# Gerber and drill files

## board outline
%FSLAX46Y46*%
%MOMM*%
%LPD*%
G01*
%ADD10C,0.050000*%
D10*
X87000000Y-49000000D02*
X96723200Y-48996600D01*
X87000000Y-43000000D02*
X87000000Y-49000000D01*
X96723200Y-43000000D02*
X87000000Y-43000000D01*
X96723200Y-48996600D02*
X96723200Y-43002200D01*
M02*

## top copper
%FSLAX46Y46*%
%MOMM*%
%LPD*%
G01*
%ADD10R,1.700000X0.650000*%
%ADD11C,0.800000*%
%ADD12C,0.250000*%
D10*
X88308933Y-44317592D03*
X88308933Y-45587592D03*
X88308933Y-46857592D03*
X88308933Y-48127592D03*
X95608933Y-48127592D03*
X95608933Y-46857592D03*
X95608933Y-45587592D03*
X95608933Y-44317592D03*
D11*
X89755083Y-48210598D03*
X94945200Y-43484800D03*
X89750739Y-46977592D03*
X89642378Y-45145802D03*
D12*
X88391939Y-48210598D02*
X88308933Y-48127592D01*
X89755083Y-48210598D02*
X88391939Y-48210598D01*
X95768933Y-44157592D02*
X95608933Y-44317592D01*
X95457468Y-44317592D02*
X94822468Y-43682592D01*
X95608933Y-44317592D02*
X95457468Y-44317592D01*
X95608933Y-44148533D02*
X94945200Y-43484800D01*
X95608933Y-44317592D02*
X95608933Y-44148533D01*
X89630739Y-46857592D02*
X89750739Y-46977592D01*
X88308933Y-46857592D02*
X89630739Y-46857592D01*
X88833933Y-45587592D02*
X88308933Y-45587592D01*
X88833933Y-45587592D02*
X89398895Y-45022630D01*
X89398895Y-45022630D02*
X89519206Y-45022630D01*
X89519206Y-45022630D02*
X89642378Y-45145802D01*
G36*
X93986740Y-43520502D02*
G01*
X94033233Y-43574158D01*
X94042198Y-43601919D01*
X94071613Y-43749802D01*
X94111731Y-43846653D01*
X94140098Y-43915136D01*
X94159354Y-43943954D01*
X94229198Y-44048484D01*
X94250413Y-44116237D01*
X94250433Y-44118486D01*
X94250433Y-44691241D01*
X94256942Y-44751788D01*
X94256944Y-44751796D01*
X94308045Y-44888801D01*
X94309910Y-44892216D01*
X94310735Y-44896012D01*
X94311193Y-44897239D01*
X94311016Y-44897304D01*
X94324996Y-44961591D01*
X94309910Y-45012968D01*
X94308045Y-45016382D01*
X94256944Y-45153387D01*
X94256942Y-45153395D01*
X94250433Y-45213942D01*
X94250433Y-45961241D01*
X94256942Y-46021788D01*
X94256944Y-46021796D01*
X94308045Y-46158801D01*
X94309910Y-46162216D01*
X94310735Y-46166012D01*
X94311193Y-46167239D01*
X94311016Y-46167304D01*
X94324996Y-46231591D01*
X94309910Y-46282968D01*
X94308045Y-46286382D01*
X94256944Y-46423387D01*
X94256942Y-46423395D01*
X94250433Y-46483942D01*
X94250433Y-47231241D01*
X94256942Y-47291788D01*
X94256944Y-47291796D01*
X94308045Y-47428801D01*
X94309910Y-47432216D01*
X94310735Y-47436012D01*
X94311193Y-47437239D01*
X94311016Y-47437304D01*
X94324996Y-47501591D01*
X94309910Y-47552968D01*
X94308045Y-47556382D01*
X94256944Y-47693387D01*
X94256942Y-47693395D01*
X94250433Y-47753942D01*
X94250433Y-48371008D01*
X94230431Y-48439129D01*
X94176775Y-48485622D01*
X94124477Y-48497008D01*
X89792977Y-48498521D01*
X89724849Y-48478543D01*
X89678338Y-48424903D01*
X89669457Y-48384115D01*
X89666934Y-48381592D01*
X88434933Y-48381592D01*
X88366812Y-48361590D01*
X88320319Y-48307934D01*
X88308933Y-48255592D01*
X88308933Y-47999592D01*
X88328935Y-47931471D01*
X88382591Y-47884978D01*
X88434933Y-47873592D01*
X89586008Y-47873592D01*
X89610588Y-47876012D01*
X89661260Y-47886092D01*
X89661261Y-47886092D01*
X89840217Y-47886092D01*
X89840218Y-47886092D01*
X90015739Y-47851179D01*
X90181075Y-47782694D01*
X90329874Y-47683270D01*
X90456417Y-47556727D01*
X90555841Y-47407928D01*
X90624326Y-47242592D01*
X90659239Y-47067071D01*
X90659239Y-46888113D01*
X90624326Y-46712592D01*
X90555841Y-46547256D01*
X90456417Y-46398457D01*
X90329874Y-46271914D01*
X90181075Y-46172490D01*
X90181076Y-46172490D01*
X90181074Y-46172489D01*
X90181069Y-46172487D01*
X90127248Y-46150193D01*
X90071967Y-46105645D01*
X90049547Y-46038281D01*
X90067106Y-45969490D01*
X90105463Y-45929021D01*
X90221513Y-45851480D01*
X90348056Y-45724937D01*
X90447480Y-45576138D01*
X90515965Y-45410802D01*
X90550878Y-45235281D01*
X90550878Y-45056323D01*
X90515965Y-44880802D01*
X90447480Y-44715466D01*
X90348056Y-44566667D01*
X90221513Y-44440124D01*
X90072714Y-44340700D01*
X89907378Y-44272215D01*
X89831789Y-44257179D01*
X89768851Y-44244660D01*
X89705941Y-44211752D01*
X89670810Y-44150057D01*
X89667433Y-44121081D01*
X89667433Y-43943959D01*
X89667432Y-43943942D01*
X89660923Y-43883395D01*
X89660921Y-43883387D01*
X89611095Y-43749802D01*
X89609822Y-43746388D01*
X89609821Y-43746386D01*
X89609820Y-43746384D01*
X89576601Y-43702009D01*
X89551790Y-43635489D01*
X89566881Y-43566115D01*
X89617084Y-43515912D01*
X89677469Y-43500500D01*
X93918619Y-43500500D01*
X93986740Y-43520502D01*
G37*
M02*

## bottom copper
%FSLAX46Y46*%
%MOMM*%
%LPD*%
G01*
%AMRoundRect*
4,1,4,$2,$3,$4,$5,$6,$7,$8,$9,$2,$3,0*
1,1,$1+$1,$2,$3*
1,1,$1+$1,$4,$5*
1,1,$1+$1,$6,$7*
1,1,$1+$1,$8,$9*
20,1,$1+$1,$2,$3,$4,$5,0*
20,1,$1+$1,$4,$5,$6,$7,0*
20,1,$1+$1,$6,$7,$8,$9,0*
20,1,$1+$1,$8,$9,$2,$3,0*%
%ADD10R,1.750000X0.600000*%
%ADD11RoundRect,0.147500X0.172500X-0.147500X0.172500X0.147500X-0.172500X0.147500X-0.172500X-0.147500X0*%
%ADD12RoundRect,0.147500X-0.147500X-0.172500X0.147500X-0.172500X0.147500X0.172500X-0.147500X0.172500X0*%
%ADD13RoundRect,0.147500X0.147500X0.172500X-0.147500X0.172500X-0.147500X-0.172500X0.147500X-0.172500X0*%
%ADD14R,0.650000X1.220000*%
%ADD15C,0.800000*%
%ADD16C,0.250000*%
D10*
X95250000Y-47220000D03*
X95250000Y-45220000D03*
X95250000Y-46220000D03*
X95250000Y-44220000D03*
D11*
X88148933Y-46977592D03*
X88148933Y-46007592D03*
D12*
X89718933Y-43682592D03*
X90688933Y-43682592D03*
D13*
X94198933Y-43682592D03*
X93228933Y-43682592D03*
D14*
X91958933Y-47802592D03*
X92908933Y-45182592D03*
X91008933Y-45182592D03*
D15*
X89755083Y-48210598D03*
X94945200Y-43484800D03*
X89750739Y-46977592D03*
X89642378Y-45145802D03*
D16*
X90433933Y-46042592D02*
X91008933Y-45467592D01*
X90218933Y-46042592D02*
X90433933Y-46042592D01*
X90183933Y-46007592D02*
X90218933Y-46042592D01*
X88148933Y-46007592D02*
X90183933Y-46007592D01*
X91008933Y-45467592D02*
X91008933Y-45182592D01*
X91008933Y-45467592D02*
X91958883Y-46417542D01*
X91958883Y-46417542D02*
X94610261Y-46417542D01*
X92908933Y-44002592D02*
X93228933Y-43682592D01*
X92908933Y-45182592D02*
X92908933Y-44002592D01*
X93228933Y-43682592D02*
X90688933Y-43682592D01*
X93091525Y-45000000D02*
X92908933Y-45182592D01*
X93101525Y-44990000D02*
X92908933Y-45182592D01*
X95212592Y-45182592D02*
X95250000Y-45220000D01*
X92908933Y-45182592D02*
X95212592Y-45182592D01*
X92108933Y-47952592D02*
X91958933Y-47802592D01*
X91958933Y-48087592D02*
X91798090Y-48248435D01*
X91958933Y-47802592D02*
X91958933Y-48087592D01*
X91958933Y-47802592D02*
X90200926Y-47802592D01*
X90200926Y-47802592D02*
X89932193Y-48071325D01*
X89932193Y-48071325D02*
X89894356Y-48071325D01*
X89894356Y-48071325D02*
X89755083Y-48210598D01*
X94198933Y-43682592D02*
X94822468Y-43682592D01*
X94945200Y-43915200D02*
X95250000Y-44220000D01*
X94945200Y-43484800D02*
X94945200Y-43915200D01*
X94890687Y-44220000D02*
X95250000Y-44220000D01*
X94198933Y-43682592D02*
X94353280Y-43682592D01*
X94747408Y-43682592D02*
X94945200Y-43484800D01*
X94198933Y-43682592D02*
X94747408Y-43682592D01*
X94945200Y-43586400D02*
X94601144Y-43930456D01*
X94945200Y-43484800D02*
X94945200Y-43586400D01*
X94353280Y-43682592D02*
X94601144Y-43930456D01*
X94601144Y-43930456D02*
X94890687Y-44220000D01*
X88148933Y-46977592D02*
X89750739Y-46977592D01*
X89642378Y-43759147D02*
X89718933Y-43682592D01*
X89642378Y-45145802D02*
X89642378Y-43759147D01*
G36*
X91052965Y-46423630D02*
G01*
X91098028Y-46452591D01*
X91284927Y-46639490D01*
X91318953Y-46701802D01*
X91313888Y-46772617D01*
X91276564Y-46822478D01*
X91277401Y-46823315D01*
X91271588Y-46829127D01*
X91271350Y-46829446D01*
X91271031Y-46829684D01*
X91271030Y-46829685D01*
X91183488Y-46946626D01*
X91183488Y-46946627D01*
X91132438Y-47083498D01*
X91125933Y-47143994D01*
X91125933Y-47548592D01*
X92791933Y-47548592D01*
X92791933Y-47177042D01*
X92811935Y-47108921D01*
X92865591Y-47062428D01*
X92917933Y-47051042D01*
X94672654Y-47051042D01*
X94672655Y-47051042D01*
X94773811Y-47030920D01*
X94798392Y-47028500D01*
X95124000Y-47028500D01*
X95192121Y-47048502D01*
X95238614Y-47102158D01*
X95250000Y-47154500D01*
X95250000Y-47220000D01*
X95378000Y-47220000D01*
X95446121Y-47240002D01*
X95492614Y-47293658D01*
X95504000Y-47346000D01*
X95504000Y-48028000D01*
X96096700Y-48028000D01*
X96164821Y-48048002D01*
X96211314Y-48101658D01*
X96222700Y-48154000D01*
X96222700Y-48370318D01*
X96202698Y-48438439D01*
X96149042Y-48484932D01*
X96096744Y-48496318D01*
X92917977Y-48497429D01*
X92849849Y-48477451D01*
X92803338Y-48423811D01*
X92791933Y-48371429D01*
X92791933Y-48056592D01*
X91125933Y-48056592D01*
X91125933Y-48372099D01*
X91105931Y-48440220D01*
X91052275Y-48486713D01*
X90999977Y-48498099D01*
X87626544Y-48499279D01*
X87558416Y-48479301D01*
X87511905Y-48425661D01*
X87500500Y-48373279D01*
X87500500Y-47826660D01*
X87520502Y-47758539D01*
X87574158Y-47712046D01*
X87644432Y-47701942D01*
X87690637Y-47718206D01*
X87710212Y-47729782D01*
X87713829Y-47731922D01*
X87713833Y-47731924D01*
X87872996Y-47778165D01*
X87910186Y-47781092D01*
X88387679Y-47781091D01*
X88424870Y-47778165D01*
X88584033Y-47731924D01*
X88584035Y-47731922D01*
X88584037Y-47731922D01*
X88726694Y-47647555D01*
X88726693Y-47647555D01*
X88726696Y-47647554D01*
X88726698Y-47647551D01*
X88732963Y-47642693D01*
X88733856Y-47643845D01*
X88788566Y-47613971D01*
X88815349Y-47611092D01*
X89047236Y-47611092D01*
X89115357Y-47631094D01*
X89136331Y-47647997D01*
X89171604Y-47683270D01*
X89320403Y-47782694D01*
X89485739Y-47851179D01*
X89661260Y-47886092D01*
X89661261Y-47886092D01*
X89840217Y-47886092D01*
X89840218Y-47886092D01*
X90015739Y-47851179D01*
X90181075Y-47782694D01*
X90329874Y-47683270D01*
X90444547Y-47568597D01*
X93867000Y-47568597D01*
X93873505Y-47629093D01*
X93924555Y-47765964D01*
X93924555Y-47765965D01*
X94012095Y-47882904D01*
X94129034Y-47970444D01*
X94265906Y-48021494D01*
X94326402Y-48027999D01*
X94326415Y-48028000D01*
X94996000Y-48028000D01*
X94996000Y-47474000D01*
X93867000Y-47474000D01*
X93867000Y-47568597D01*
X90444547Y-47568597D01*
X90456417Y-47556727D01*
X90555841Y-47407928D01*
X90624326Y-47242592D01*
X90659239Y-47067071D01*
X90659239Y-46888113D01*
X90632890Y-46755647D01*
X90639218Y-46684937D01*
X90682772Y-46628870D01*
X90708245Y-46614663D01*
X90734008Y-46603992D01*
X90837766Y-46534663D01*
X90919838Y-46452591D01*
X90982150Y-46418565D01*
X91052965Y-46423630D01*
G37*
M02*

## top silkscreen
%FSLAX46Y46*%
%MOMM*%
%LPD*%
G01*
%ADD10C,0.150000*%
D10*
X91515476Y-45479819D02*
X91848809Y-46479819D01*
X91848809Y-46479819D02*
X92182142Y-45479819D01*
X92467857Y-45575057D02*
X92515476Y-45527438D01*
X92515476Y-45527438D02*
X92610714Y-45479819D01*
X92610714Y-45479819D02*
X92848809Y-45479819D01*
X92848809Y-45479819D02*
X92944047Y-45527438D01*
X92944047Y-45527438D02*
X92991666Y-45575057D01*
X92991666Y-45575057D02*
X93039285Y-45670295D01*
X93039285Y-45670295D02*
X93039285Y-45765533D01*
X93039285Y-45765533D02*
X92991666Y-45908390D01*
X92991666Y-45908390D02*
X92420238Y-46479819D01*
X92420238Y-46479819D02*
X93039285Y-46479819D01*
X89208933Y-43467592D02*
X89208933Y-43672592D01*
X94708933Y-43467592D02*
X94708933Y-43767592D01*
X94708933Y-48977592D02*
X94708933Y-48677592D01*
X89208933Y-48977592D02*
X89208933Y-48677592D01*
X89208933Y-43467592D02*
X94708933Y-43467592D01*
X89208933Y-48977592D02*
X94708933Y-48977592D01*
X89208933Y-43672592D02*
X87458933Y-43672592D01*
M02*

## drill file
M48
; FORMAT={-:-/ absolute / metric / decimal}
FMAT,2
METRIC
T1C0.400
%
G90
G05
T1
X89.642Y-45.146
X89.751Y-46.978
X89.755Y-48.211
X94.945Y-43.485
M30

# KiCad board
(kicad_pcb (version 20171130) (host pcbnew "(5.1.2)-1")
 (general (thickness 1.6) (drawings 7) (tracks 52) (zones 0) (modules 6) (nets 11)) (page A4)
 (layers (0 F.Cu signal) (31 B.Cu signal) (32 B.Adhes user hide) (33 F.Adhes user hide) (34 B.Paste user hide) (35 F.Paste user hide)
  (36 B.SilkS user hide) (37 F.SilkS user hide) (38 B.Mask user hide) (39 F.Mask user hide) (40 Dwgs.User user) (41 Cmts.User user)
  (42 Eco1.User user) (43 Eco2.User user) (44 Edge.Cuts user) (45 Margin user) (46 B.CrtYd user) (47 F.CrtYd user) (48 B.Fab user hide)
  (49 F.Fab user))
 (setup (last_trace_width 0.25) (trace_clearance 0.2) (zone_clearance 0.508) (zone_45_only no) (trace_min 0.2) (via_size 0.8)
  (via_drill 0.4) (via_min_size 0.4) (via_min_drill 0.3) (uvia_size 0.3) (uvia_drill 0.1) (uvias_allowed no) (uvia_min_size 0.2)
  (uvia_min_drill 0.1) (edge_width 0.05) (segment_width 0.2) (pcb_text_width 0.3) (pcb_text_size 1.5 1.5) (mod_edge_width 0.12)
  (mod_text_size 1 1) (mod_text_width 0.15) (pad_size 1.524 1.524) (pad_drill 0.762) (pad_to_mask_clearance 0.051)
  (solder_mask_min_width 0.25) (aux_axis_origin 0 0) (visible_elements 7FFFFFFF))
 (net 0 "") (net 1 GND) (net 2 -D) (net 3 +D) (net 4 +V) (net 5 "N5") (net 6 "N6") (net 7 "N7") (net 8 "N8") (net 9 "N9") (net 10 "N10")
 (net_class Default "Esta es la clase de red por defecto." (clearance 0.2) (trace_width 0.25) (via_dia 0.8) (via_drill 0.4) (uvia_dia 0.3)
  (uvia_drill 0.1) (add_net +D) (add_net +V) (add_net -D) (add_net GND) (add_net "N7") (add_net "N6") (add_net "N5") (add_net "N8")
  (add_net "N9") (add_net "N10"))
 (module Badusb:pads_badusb (layer B.Cu) (at 93.98 45.72 180)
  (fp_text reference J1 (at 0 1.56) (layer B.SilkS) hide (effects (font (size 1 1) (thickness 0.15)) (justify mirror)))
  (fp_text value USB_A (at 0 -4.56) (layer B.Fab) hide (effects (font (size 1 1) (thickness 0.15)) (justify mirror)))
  (pad 4 smd rect (at -1.27 -1.5 180) (size 1.75 0.6) (layers B.Cu B.Paste B.Mask) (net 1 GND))
  (pad 2 smd rect (at -1.27 0.5 180) (size 1.75 0.6) (layers B.Cu B.Paste B.Mask) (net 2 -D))
  (pad 3 smd rect (at -1.27 -0.5 180) (size 1.75 0.6) (layers B.Cu B.Paste B.Mask) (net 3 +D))
  (pad 1 smd rect (at -1.27 1.5 180) (size 1.75 0.6) (layers B.Cu B.Paste B.Mask) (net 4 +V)))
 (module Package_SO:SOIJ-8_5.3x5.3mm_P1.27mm (layer F.Cu) (at 91.958933 46.222592)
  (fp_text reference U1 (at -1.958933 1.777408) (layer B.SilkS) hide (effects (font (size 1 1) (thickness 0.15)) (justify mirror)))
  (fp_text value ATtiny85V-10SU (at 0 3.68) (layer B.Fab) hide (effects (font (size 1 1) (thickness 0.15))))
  (fp_line (start -2.75 -2.755) (end -2.75 -2.55) (layer F.SilkS) (width 0.15))
  (fp_line (start 2.75 -2.755) (end 2.75 -2.455) (layer F.SilkS) (width 0.15))
  (fp_line (start 2.75 2.755) (end 2.75 2.455) (layer F.SilkS) (width 0.15))
  (fp_line (start -2.75 2.755) (end -2.75 2.455) (layer F.SilkS) (width 0.15))
  (fp_line (start -2.75 -2.755) (end 2.75 -2.755) (layer F.SilkS) (width 0.15))
  (fp_line (start -2.75 2.755) (end 2.75 2.755) (layer F.SilkS) (width 0.15))
  (fp_line (start -2.75 -2.55) (end -4.5 -2.55) (layer F.SilkS) (width 0.15))
  (pad 1 smd rect (at -3.65 -1.905) (size 1.7 0.65) (layers F.Cu F.Paste F.Mask) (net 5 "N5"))
  (pad 2 smd rect (at -3.65 -0.635) (size 1.7 0.65) (layers F.Cu F.Paste F.Mask) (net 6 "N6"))
  (pad 3 smd rect (at -3.65 0.635) (size 1.7 0.65) (layers F.Cu F.Paste F.Mask) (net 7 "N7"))
  (pad 4 smd rect (at -3.65 1.905) (size 1.7 0.65) (layers F.Cu F.Paste F.Mask) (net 1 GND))
  (pad 5 smd rect (at 3.65 1.905) (size 1.7 0.65) (layers F.Cu F.Paste F.Mask) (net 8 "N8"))
  (pad 6 smd rect (at 3.65 0.635) (size 1.7 0.65) (layers F.Cu F.Paste F.Mask) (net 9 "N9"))
  (pad 7 smd rect (at 3.65 -0.635) (size 1.7 0.65) (layers F.Cu F.Paste F.Mask) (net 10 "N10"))
  (pad 8 smd rect (at 3.65 -1.905) (size 1.7 0.65) (layers F.Cu F.Paste F.Mask) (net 4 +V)))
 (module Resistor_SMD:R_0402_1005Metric (layer B.Cu) (at 88.148933 46.492592 90)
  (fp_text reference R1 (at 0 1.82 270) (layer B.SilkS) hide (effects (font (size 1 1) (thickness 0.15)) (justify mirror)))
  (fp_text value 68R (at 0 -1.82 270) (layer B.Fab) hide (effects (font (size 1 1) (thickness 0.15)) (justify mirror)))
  (pad 1 smd roundrect (at -0.485 0 90) (size 0.59 0.64) (layers B.Cu B.Paste B.Mask) (roundrect_rratio 0.25) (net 7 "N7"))
  (pad 2 smd roundrect (at 0.485 0 90) (size 0.59 0.64) (layers B.Cu B.Paste B.Mask) (roundrect_rratio 0.25) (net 3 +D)))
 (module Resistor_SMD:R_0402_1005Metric (layer B.Cu) (at 90.203933 43.682592)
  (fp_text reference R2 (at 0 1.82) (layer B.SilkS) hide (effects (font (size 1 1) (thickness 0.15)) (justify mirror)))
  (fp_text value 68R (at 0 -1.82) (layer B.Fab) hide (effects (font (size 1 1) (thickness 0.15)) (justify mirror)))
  (pad 1 smd roundrect (at -0.485 0) (size 0.59 0.64) (layers B.Cu B.Paste B.Mask) (roundrect_rratio 0.25) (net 6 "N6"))
  (pad 2 smd roundrect (at 0.485 0) (size 0.59 0.64) (layers B.Cu B.Paste B.Mask) (roundrect_rratio 0.25) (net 2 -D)))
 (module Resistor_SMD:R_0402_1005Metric (layer B.Cu) (at 93.713933 43.682592 180)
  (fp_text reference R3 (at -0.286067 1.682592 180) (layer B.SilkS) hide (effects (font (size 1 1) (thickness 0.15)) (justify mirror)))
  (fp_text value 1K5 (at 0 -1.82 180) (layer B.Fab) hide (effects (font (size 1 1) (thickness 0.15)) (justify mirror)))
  (pad 1 smd roundrect (at -0.485 0 180) (size 0.59 0.64) (layers B.Cu B.Paste B.Mask) (roundrect_rratio 0.25) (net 4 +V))
  (pad 2 smd roundrect (at 0.485 0 180) (size 0.59 0.64) (layers B.Cu B.Paste B.Mask) (roundrect_rratio 0.25) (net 2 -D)))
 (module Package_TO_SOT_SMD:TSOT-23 (layer B.Cu) (at 91.958933 46.492592 270)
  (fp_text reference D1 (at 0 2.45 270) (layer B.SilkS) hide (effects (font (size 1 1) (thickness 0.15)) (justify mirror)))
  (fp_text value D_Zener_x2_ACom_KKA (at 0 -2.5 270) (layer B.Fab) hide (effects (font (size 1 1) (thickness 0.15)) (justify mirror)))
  (pad 3 smd rect (at 1.31 0 270) (size 1.22 0.65) (layers B.Cu B.Paste B.Mask) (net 1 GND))
  (pad 2 smd rect (at -1.31 -0.95 270) (size 1.22 0.65) (layers B.Cu B.Paste B.Mask) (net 2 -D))
  (pad 1 smd rect (at -1.31 0.95 270) (size 1.22 0.65) (layers B.Cu B.Paste B.Mask) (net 3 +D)))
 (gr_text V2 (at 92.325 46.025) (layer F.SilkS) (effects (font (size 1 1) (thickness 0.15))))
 (gr_line (start 87 49) (end 96.7232 48.9966) (layer Edge.Cuts) (width 0.05))
 (gr_line (start 87 43) (end 87 49) (layer Edge.Cuts) (width 0.05))
 (gr_line (start 96.7232 43) (end 87 43) (layer Edge.Cuts) (width 0.05))
 (gr_line (start 96.7232 48.9966) (end 96.7232 43.0022) (layer Edge.Cuts) (width 0.05))
 (segment (start 90.433933 46.042592) (end 91.008933 45.467592) (width 0.25) (layer B.Cu) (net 3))
 (segment (start 90.218933 46.042592) (end 90.433933 46.042592) (width 0.25) (layer B.Cu) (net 3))
 (segment (start 90.183933 46.007592) (end 90.218933 46.042592) (width 0.25) (layer B.Cu) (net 3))
 (segment (start 88.148933 46.007592) (end 90.183933 46.007592) (width 0.25) (layer B.Cu) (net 3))
 (segment (start 91.008933 45.467592) (end 91.008933 45.182592) (width 0.25) (layer B.Cu) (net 3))
 (segment (start 91.008933 45.467592) (end 91.958883 46.417542) (width 0.25) (layer B.Cu) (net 3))
 (segment (start 91.958883 46.417542) (end 94.610261 46.417542) (width 0.25) (layer B.Cu) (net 3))
 (segment (start 92.908933 44.002592) (end 93.228933 43.682592) (width 0.25) (layer B.Cu) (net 2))
 (segment (start 92.908933 45.182592) (end 92.908933 44.002592) (width 0.25) (layer B.Cu) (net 2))
 (segment (start 93.228933 43.682592) (end 90.688933 43.682592) (width 0.25) (layer B.Cu) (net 2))
 (segment (start 93.091525 45) (end 92.908933 45.182592) (width 0.25) (layer B.Cu) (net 2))
 (segment (start 93.101525 44.99) (end 92.908933 45.182592) (width 0.25) (layer B.Cu) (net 2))
 (segment (start 95.212592 45.182592) (end 95.25 45.22) (width 0.25) (layer B.Cu) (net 2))
 (segment (start 92.908933 45.182592) (end 95.212592 45.182592) (width 0.25) (layer B.Cu) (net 2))
 (segment (start 92.108933 47.952592) (end 91.958933 47.802592) (width 0.25) (layer B.Cu) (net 1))
 (segment (start 91.958933 48.087592) (end 91.79809 48.248435) (width 0.25) (layer B.Cu) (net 1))
 (segment (start 91.958933 47.802592) (end 91.958933 48.087592) (width 0.25) (layer B.Cu) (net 1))
 (segment (start 91.958933 47.802592) (end 90.200926 47.802592) (width 0.25) (layer B.Cu) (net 1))
 (segment (start 90.200926 47.802592) (end 89.932193 48.071325) (width 0.25) (layer B.Cu) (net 1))
 (via (at 89.755083 48.210598) (size 0.8) (drill 0.4) (layers F.Cu B.Cu) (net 1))
 (segment (start 89.932193 48.071325) (end 89.894356 48.071325) (width 0.25) (layer B.Cu) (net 1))
 (segment (start 89.894356 48.071325) (end 89.755083 48.210598) (width 0.25) (layer B.Cu) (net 1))
 (segment (start 88.391939 48.210598) (end 88.308933 48.127592) (width 0.25) (layer F.Cu) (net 1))
 (segment (start 89.755083 48.210598) (end 88.391939 48.210598) (width 0.25) (layer F.Cu) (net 1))
 (segment (start 95.768933 44.157592) (end 95.608933 44.317592) (width 0.25) (layer F.Cu) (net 4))
 (segment (start 94.198933 43.682592) (end 94.822468 43.682592) (width 0.25) (layer B.Cu) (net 4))
 (via (at 94.9452 43.4848) (size 0.8) (drill 0.4) (layers F.Cu B.Cu) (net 4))
 (segment (start 95.457468 44.317592) (end 94.822468 43.682592) (width 0.25) (layer F.Cu) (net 4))
 (segment (start 95.608933 44.317592) (end 95.457468 44.317592) (width 0.25) (layer F.Cu) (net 4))
 (segment (start 95.608933 44.148533) (end 94.9452 43.4848) (width 0.25) (layer F.Cu) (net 4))
 (segment (start 95.608933 44.317592) (end 95.608933 44.148533) (width 0.25) (layer F.Cu) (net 4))
 (segment (start 94.9452 43.9152) (end 95.25 44.22) (width 0.25) (layer B.Cu) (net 4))
 (segment (start 94.9452 43.4848) (end 94.9452 43.9152) (width 0.25) (layer B.Cu) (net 4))
 (segment (start 94.890687 44.22) (end 95.25 44.22) (width 0.25) (layer B.Cu) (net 4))
 (segment (start 94.198933 43.682592) (end 94.35328 43.682592) (width 0.25) (layer B.Cu) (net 4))
 (segment (start 94.747408 43.682592) (end 94.9452 43.4848) (width 0.25) (layer B.Cu) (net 4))
 (segment (start 94.198933 43.682592) (end 94.747408 43.682592) (width 0.25) (layer B.Cu) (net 4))
 (segment (start 94.9452 43.5864) (end 94.601144 43.930456) (width 0.25) (layer B.Cu) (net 4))
 (segment (start 94.9452 43.4848) (end 94.9452 43.5864) (width 0.25) (layer B.Cu) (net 4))
 (segment (start 94.35328 43.682592) (end 94.601144 43.930456) (width 0.25) (layer B.Cu) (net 4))
 (segment (start 94.601144 43.930456) (end 94.890687 44.22) (width 0.25) (layer B.Cu) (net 4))
 (segment (start 88.148933 46.977592) (end 89.750739 46.977592) (width 0.25) (layer B.Cu) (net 7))
 (via (at 89.750739 46.977592) (size 0.8) (drill 0.4) (layers F.Cu B.Cu) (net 7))
 (segment (start 89.630739 46.857592) (end 89.750739 46.977592) (width 0.25) (layer F.Cu) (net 7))
 (segment (start 88.308933 46.857592) (end 89.630739 46.857592) (width 0.25) (layer F.Cu) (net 7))
 (segment (start 88.833933 45.587592) (end 88.308933 45.587592) (width 0.25) (layer F.Cu) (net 6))
 (segment (start 88.833933 45.587592) (end 89.398895 45.02263) (width 0.25) (layer F.Cu) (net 6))
 (via (at 89.642378 45.145802) (size 0.8) (drill 0.4) (layers F.Cu B.Cu) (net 6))
 (segment (start 89.398895 45.02263) (end 89.519206 45.02263) (width 0.25) (layer F.Cu) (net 6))
 (segment (start 89.519206 45.02263) (end 89.642378 45.145802) (width 0.25) (layer F.Cu) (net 6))
 (segment (start 89.642378 43.759147) (end 89.718933 43.682592) (width 0.25) (layer B.Cu) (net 6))
 (segment (start 89.642378 45.145802) (end 89.642378 43.759147) (width 0.25) (layer B.Cu) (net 6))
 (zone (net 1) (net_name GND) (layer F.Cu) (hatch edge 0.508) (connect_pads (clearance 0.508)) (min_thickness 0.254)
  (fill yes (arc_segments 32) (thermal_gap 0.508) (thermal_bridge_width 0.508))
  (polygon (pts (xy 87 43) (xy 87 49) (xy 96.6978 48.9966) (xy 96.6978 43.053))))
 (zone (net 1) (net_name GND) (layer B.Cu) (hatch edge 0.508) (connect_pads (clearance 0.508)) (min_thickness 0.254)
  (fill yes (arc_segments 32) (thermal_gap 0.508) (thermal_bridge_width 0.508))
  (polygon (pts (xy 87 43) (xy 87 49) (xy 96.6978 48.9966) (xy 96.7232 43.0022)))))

